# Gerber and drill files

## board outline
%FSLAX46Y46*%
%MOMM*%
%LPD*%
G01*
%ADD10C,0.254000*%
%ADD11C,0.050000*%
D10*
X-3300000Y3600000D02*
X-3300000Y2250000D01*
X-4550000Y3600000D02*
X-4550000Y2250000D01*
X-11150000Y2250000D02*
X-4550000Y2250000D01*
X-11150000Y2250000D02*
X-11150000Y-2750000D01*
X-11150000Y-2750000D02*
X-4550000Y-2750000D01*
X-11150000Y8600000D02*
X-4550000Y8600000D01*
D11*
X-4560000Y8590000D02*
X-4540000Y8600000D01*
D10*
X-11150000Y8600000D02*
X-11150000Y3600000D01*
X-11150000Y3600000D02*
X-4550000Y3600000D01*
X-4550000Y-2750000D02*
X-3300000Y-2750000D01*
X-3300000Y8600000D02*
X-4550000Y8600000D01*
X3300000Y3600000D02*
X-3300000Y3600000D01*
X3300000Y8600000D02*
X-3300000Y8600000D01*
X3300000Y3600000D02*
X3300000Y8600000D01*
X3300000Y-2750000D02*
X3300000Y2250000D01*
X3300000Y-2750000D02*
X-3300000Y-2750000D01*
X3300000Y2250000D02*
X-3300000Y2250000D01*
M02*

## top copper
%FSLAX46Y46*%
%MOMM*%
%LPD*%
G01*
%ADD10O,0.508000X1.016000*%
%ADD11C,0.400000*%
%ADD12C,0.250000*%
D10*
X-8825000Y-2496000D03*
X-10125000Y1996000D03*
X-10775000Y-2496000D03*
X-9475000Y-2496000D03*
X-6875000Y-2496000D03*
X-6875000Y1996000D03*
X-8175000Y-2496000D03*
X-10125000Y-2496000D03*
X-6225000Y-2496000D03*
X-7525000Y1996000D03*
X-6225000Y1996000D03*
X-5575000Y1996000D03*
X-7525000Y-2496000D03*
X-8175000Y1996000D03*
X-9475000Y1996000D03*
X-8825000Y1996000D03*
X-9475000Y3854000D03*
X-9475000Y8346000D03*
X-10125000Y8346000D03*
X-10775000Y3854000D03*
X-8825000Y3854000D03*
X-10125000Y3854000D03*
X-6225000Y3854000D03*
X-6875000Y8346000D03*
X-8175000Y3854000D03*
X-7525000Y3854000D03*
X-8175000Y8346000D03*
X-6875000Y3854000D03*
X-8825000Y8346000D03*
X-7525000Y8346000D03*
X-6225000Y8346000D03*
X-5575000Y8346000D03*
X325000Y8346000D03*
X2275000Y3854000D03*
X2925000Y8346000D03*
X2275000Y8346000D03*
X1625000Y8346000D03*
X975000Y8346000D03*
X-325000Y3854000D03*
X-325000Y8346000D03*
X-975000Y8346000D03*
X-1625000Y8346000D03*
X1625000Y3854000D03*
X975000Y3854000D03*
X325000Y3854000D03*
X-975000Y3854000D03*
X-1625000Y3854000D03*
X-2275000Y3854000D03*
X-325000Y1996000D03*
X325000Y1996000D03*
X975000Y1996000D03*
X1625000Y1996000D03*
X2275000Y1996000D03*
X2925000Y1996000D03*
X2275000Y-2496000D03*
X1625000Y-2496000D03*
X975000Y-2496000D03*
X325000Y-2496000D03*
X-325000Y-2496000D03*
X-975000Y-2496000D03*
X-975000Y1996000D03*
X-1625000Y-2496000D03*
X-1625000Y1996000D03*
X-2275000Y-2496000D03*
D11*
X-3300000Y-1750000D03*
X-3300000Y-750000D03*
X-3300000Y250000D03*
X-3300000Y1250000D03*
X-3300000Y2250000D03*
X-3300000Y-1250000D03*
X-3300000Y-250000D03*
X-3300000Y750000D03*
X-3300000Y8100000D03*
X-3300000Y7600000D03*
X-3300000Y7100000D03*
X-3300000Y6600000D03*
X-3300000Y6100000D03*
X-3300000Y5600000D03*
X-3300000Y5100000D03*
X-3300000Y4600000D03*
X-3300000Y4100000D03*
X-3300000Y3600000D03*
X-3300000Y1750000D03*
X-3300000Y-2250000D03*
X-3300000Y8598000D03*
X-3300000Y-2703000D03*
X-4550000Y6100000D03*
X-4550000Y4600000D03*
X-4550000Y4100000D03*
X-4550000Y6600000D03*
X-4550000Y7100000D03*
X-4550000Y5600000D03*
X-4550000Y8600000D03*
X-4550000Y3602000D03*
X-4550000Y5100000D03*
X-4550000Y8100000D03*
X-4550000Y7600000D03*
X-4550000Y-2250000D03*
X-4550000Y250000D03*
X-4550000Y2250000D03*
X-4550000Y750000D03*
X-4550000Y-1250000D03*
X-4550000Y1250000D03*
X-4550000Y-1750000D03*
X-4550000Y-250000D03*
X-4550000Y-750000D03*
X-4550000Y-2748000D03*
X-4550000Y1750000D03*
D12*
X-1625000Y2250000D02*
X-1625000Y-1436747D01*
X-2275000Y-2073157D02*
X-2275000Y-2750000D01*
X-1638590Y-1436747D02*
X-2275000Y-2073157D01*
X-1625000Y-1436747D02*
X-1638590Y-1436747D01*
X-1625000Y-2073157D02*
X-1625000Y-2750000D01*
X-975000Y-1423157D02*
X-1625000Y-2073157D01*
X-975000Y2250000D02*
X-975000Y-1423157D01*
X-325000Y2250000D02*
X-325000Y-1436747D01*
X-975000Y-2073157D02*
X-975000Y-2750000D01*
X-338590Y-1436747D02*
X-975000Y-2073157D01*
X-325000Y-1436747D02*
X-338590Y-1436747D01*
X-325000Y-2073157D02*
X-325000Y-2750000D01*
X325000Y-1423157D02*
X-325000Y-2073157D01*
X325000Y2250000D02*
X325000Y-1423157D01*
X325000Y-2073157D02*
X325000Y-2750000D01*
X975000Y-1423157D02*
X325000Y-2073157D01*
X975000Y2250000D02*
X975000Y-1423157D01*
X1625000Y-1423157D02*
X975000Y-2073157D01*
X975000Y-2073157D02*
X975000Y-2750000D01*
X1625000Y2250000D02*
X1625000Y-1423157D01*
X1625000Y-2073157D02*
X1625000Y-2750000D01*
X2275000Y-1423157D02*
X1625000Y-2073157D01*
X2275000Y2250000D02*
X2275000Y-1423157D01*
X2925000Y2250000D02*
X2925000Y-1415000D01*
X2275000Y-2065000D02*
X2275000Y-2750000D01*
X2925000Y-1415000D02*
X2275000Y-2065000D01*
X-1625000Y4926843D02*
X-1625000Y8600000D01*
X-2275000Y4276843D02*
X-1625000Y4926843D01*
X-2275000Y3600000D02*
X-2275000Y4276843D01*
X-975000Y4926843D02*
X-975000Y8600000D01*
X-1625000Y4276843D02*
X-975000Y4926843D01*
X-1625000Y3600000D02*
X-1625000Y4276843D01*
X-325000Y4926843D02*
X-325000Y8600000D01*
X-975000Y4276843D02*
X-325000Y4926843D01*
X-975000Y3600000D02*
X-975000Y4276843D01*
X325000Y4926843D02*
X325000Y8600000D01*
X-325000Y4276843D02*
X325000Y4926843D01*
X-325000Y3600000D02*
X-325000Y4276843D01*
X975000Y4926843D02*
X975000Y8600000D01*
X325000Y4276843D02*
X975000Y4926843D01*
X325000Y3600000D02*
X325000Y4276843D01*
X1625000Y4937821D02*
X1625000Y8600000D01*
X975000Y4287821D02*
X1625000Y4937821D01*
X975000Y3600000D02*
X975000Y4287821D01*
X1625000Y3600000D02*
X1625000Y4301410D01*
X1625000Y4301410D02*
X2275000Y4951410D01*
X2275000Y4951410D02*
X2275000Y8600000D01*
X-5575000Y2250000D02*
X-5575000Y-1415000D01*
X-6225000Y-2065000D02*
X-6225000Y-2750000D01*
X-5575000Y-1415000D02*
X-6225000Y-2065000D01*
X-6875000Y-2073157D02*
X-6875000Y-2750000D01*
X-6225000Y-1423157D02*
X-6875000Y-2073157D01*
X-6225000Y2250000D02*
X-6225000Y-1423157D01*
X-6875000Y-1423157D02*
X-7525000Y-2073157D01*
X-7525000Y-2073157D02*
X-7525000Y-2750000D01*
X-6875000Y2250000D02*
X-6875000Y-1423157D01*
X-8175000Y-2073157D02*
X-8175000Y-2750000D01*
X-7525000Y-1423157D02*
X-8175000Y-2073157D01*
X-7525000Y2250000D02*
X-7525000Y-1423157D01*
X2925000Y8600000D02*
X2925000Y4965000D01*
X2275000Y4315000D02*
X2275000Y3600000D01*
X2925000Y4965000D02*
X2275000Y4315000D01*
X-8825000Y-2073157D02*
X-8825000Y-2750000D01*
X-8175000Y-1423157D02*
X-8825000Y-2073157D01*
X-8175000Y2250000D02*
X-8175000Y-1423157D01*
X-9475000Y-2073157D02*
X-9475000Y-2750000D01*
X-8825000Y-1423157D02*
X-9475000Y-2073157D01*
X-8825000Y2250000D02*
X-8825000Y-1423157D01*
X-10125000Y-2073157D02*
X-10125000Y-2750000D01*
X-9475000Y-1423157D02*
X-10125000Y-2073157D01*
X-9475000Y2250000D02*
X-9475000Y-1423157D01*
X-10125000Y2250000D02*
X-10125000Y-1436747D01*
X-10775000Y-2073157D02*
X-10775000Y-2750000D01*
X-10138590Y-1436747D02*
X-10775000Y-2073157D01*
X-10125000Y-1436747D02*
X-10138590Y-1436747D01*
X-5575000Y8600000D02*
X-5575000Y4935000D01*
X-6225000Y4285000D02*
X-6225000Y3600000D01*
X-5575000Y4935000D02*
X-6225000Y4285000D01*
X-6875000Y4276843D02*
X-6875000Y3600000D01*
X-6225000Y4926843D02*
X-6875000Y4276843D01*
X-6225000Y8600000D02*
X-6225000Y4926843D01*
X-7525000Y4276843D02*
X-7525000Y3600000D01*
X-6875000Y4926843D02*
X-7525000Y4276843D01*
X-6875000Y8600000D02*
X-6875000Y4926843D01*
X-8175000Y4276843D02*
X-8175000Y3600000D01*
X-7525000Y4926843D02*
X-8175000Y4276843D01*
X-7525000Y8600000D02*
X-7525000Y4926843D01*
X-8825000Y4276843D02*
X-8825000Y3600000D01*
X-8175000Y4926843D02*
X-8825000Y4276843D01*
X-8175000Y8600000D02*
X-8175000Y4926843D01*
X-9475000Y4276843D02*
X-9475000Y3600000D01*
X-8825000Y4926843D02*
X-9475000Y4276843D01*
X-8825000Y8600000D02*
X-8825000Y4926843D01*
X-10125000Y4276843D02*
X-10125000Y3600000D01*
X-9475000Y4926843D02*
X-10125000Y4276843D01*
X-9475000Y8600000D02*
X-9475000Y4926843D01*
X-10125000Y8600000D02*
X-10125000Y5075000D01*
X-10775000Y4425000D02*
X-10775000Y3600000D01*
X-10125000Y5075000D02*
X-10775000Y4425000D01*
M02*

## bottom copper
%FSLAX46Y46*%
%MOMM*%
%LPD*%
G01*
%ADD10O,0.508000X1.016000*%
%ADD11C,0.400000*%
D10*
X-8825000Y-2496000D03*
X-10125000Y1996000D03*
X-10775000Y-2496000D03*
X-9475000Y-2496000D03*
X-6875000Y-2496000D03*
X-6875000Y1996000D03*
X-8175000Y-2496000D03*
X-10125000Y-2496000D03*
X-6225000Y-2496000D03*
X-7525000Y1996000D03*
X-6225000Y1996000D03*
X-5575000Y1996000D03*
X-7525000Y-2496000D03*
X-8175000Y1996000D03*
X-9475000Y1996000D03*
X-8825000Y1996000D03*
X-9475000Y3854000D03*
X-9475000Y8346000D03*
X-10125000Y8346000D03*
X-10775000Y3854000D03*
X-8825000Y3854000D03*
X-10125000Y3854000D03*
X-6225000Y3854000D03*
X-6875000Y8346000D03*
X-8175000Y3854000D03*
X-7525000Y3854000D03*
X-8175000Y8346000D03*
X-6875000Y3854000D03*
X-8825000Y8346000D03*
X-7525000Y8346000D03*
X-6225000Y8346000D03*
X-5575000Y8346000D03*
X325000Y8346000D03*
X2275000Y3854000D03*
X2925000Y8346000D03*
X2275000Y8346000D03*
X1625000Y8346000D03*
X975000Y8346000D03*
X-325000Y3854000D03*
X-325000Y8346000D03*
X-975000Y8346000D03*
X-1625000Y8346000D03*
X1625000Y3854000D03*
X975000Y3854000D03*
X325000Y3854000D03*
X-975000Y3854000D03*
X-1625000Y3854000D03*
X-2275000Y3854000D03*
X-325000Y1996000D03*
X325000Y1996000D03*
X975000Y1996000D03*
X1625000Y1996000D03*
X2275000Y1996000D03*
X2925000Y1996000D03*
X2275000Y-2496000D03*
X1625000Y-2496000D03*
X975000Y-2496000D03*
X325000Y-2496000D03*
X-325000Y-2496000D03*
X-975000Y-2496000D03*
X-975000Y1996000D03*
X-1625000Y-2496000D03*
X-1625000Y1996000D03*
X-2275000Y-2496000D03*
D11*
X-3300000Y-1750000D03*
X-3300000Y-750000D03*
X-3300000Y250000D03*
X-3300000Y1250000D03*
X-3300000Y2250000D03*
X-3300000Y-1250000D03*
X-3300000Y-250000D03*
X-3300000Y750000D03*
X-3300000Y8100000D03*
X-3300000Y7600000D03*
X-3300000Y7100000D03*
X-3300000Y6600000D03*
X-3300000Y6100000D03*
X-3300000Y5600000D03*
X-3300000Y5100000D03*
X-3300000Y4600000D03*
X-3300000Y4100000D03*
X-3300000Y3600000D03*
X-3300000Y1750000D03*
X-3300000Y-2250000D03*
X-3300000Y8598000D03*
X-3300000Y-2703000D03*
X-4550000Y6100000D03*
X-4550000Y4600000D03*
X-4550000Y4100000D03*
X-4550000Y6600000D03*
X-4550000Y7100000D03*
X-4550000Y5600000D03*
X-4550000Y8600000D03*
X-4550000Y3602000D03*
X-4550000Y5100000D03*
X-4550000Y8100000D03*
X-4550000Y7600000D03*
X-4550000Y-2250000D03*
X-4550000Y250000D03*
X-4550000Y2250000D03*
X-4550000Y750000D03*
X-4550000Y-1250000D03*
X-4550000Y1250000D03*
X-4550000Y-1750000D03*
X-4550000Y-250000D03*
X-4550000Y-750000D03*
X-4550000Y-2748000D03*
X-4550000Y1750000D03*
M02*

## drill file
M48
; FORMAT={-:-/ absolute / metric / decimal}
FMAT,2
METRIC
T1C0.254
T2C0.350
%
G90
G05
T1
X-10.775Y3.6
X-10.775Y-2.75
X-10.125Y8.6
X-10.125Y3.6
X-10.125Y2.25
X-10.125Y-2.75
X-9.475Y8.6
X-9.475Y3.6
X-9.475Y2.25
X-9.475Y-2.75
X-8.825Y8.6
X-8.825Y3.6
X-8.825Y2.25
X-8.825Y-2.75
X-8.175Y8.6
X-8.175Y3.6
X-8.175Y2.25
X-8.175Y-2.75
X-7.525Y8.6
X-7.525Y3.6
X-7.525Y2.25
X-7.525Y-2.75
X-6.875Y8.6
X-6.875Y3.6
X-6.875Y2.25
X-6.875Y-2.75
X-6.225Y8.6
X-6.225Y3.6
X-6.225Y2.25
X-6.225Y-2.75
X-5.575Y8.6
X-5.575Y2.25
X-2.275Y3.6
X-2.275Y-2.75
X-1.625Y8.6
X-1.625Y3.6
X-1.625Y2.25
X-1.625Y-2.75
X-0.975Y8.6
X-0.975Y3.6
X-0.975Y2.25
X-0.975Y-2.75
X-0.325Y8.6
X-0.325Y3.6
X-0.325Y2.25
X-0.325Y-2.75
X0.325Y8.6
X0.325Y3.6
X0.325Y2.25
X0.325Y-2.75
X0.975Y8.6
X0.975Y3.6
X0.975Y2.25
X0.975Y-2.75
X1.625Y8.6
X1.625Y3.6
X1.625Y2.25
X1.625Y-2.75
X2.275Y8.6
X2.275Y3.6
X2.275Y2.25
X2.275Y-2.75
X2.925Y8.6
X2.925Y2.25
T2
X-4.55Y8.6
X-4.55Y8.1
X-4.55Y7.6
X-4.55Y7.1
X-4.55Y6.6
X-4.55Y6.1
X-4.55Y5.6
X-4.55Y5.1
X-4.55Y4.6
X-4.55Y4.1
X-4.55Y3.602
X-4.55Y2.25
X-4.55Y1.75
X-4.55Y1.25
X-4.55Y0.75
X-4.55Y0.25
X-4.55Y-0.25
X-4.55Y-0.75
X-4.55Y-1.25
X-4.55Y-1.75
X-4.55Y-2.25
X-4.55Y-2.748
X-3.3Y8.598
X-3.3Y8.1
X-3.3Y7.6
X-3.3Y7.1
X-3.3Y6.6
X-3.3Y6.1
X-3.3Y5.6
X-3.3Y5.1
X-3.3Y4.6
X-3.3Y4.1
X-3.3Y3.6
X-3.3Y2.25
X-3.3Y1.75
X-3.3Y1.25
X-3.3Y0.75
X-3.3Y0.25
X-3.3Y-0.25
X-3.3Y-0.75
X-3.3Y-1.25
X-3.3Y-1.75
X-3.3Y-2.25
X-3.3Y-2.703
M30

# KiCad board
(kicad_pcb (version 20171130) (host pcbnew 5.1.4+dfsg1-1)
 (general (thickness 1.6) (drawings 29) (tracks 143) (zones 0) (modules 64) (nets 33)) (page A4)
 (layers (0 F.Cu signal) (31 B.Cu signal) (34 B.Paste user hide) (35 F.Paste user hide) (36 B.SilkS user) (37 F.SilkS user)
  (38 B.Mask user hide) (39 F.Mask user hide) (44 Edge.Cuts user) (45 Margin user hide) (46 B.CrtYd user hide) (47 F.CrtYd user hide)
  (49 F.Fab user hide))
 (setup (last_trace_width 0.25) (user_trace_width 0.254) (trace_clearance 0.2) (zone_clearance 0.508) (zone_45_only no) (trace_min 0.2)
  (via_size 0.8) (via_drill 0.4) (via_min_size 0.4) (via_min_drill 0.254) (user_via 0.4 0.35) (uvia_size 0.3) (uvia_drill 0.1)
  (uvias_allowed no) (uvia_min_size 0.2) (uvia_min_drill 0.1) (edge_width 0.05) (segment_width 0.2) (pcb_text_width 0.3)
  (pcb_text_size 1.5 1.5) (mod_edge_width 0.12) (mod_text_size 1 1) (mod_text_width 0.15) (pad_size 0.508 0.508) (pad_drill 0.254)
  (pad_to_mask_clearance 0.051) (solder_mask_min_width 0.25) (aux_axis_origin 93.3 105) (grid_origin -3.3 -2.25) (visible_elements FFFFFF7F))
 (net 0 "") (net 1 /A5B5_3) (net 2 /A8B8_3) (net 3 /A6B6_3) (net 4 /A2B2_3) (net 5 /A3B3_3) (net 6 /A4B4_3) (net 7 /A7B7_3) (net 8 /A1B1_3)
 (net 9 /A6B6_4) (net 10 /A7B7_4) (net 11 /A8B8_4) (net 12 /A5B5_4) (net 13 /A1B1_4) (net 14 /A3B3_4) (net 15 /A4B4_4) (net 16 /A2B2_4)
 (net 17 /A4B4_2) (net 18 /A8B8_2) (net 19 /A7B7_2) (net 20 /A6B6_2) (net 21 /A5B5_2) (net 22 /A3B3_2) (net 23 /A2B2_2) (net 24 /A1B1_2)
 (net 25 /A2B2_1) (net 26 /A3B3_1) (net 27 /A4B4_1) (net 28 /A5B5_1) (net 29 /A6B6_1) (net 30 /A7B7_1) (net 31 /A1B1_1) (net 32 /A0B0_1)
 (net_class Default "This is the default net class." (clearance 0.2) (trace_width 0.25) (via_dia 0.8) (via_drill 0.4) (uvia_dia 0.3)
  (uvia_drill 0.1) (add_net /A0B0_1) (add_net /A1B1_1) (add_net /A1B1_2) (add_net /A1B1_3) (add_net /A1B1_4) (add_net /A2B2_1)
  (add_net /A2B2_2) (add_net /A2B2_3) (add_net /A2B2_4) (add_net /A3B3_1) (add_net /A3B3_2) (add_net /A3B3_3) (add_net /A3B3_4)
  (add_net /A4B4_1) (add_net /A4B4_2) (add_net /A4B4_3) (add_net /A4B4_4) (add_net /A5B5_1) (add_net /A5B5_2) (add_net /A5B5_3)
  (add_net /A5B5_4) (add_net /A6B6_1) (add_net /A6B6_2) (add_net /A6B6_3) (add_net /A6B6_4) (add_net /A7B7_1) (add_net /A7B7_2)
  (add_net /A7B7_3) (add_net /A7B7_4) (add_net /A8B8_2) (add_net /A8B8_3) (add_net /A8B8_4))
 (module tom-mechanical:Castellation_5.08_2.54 (layer F.Cu) (at -8.825 2.75 180)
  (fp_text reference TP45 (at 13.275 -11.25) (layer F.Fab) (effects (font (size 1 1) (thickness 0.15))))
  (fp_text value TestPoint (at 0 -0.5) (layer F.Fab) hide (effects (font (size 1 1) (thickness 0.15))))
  (pad 1 thru_hole oval (at 0 0 180) (size 0.508 1.016) (drill 0.254 (offset 0 0.254)) (layers *.Cu *.Mask) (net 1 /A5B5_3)))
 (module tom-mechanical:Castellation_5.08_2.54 (layer F.Cu) (at -10.125 -2.25)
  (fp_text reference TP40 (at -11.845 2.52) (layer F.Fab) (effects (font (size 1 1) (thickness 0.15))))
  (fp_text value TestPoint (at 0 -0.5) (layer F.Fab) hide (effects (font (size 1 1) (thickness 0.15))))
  (pad 1 thru_hole oval (at 0 0) (size 0.508 1.016) (drill 0.254 (offset 0 0.254)) (layers *.Cu *.Mask) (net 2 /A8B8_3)))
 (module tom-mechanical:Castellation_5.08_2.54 (layer F.Cu) (at -10.775 2.75 180)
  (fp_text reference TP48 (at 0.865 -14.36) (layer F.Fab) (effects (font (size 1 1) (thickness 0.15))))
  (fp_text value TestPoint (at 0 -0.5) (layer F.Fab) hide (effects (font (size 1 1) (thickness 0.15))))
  (pad 1 thru_hole oval (at 0 0 180) (size 0.508 1.016) (drill 0.254 (offset 0 0.254)) (layers *.Cu *.Mask) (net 2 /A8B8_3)))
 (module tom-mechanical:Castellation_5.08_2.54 (layer F.Cu) (at -9.475 2.75 180)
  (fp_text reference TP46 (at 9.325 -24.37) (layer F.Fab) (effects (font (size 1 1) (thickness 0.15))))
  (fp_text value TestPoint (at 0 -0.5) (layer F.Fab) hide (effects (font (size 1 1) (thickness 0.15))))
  (pad 1 thru_hole oval (at 0 0 180) (size 0.508 1.016) (drill 0.254 (offset 0 0.254)) (layers *.Cu *.Mask) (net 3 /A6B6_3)))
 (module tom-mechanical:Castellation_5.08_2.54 (layer F.Cu) (at -6.875 2.75 180)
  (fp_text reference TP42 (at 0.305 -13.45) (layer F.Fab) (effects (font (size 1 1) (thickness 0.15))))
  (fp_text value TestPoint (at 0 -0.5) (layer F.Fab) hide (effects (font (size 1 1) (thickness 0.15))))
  (pad 1 thru_hole oval (at 0 0 180) (size 0.508 1.016) (drill 0.254 (offset 0 0.254)) (layers *.Cu *.Mask) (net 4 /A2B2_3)))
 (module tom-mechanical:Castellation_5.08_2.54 (layer F.Cu) (at -6.875 -2.25)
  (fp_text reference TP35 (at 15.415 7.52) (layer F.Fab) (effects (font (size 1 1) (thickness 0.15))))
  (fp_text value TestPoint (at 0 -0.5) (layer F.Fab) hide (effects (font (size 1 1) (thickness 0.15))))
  (pad 1 thru_hole oval (at 0 0) (size 0.508 1.016) (drill 0.254 (offset 0 0.254)) (layers *.Cu *.Mask) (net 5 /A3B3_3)))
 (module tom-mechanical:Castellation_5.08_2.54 (layer F.Cu) (at -8.175 2.75 180)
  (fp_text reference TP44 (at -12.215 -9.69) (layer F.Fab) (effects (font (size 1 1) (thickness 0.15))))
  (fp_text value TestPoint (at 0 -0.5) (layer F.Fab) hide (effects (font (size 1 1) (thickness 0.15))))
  (pad 1 thru_hole oval (at 0 0 180) (size 0.508 1.016) (drill 0.254 (offset 0 0.254)) (layers *.Cu *.Mask) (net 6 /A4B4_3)))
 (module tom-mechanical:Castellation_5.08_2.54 (layer F.Cu) (at -10.125 2.75 180)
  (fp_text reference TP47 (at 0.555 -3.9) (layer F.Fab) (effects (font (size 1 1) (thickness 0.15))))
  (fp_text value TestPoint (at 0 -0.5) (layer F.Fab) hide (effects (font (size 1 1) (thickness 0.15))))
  (pad 1 thru_hole oval (at 0 0 180) (size 0.508 1.016) (drill 0.254 (offset 0 0.254)) (layers *.Cu *.Mask) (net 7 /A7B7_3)))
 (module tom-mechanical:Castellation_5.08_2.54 (layer F.Cu) (at -6.225 2.75 180)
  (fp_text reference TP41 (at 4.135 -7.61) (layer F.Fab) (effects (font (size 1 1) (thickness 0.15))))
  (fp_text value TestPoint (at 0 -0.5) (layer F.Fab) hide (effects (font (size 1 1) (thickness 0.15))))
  (pad 1 thru_hole oval (at 0 0 180) (size 0.508 1.016) (drill 0.254 (offset 0 0.254)) (layers *.Cu *.Mask) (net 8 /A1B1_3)))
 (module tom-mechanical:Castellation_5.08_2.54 (layer F.Cu) (at -7.525 -2.25)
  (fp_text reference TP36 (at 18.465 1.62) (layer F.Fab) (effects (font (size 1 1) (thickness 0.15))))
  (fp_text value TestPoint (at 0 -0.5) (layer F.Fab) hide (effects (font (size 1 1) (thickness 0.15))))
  (pad 1 thru_hole oval (at 0 0) (size 0.508 1.016) (drill 0.254 (offset 0 0.254)) (layers *.Cu *.Mask) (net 6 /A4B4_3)))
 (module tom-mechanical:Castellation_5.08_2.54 (layer F.Cu) (at -6.225 -2.25)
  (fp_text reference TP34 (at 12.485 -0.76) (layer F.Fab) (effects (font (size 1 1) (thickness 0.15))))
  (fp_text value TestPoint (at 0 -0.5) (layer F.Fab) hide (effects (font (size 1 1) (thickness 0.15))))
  (pad 1 thru_hole oval (at 0 0) (size 0.508 1.016) (drill 0.254 (offset 0 0.254)) (layers *.Cu *.Mask) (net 4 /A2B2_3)))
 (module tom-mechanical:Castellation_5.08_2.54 (layer F.Cu) (at -5.575 -2.25)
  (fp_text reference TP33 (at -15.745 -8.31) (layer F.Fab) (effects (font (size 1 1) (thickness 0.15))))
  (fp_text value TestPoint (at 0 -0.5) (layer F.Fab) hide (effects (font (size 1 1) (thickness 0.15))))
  (pad 1 thru_hole oval (at 0 0) (size 0.508 1.016) (drill 0.254 (offset 0 0.254)) (layers *.Cu *.Mask) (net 8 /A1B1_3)))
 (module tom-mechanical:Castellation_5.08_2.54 (layer F.Cu) (at -7.525 2.75 180)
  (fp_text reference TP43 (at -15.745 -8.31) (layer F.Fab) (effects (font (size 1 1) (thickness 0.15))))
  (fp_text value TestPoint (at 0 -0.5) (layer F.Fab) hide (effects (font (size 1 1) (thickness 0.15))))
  (pad 1 thru_hole oval (at 0 0 180) (size 0.508 1.016) (drill 0.254 (offset 0 0.254)) (layers *.Cu *.Mask) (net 5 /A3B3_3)))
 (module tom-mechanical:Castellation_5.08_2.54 (layer F.Cu) (at -8.175 -2.25)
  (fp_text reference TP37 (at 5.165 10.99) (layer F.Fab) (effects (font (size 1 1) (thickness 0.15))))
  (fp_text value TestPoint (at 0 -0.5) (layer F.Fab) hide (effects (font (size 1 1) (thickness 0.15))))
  (pad 1 thru_hole oval (at 0 0) (size 0.508 1.016) (drill 0.254 (offset 0 0.254)) (layers *.Cu *.Mask) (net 1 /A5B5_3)))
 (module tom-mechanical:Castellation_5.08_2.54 (layer F.Cu) (at -9.475 -2.25)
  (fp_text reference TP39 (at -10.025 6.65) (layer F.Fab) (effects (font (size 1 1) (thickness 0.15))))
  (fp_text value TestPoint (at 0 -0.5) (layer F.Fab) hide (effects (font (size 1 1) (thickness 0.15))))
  (pad 1 thru_hole oval (at 0 0) (size 0.508 1.016) (drill 0.254 (offset 0 0.254)) (layers *.Cu *.Mask) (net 7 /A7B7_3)))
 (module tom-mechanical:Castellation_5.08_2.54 (layer F.Cu) (at -8.825 -2.25)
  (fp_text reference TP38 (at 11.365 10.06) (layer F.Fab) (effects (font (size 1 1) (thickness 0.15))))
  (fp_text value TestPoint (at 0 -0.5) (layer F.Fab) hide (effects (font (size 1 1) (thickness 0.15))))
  (pad 1 thru_hole oval (at 0 0) (size 0.508 1.016) (drill 0.254 (offset 0 0.254)) (layers *.Cu *.Mask) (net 3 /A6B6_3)))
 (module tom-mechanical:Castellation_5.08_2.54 (layer F.Cu) (at -9.475 -3.6 180)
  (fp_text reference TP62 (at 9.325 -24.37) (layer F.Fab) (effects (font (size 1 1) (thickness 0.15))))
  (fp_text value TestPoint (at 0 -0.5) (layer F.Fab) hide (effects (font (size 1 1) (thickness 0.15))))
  (pad 1 thru_hole oval (at 0 0 180) (size 0.508 1.016) (drill 0.254 (offset 0 0.254)) (layers *.Cu *.Mask) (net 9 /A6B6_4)))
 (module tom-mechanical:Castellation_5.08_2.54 (layer F.Cu) (at -9.475 -8.6)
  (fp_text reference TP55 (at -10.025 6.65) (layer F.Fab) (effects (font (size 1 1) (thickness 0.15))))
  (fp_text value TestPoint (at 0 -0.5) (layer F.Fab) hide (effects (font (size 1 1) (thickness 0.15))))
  (pad 1 thru_hole oval (at 0 0) (size 0.508 1.016) (drill 0.254 (offset 0 0.254)) (layers *.Cu *.Mask) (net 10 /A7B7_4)))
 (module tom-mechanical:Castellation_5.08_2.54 (layer F.Cu) (at -10.125 -8.6)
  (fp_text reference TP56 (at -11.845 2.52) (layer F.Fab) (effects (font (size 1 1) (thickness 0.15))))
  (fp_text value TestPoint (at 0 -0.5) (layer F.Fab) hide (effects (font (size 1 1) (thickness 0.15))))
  (pad 1 thru_hole oval (at 0 0) (size 0.508 1.016) (drill 0.254 (offset 0 0.254)) (layers *.Cu *.Mask) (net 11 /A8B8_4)))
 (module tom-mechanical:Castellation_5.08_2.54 (layer F.Cu) (at -10.775 -3.6 180)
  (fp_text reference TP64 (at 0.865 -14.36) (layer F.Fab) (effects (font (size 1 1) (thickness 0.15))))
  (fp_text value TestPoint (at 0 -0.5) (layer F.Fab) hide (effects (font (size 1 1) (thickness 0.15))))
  (pad 1 thru_hole oval (at 0 0 180) (size 0.508 1.016) (drill 0.254 (offset 0 0.254)) (layers *.Cu *.Mask) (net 11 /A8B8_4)))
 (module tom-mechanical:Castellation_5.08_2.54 (layer F.Cu) (at -8.825 -3.6 180)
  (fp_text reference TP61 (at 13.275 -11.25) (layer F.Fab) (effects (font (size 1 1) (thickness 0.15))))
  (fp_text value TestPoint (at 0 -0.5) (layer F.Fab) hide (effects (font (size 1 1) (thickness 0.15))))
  (pad 1 thru_hole oval (at 0 0 180) (size 0.508 1.016) (drill 0.254 (offset 0 0.254)) (layers *.Cu *.Mask) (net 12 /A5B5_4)))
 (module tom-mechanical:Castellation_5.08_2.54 (layer F.Cu) (at -10.125 -3.6 180)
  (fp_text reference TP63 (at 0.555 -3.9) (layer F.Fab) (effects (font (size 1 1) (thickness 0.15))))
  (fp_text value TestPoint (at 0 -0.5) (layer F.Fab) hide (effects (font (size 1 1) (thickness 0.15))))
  (pad 1 thru_hole oval (at 0 0 180) (size 0.508 1.016) (drill 0.254 (offset 0 0.254)) (layers *.Cu *.Mask) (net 10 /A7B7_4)))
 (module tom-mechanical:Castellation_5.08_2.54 (layer F.Cu) (at -6.225 -3.6 180)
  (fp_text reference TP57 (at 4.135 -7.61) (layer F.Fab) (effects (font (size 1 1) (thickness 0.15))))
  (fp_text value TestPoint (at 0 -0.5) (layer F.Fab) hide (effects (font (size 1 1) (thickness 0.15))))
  (pad 1 thru_hole oval (at 0 0 180) (size 0.508 1.016) (drill 0.254 (offset 0 0.254)) (layers *.Cu *.Mask) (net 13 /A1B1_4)))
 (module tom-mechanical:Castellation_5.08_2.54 (layer F.Cu) (at -6.875 -8.6)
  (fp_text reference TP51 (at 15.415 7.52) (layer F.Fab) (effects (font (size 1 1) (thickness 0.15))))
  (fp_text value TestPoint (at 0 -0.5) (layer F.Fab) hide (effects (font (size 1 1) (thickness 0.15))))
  (pad 1 thru_hole oval (at 0 0) (size 0.508 1.016) (drill 0.254 (offset 0 0.254)) (layers *.Cu *.Mask) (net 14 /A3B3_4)))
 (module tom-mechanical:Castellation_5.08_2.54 (layer F.Cu) (at -8.175 -3.6 180)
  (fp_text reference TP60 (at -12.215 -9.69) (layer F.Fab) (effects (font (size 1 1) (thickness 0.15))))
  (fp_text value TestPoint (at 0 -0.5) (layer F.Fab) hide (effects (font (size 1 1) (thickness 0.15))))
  (pad 1 thru_hole oval (at 0 0 180) (size 0.508 1.016) (drill 0.254 (offset 0 0.254)) (layers *.Cu *.Mask) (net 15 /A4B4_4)))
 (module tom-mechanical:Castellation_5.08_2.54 (layer F.Cu) (at -7.525 -3.6 180)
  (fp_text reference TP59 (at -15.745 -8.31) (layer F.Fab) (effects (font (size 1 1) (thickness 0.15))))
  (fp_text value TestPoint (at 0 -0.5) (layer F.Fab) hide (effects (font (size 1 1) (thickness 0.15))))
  (pad 1 thru_hole oval (at 0 0 180) (size 0.508 1.016) (drill 0.254 (offset 0 0.254)) (layers *.Cu *.Mask) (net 14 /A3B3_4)))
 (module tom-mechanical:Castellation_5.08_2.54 (layer F.Cu) (at -8.175 -8.6)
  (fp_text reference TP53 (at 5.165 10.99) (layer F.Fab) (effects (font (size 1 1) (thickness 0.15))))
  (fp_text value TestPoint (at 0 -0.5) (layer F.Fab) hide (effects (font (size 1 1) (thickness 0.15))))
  (pad 1 thru_hole oval (at 0 0) (size 0.508 1.016) (drill 0.254 (offset 0 0.254)) (layers *.Cu *.Mask) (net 12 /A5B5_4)))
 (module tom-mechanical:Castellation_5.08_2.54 (layer F.Cu) (at -6.875 -3.6 180)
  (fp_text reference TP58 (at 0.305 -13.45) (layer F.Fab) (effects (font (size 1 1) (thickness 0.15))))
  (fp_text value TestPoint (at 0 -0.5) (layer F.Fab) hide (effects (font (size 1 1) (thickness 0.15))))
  (pad 1 thru_hole oval (at 0 0 180) (size 0.508 1.016) (drill 0.254 (offset 0 0.254)) (layers *.Cu *.Mask) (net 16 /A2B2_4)))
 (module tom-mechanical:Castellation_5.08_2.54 (layer F.Cu) (at -8.825 -8.6)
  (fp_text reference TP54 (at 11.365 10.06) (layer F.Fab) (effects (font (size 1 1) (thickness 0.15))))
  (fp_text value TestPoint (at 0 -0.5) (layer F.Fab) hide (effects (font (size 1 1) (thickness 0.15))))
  (pad 1 thru_hole oval (at 0 0) (size 0.508 1.016) (drill 0.254 (offset 0 0.254)) (layers *.Cu *.Mask) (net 9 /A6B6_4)))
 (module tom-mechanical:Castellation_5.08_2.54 (layer F.Cu) (at -7.525 -8.6)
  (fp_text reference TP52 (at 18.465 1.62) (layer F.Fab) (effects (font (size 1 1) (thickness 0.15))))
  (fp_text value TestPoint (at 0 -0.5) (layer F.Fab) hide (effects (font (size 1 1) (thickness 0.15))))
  (pad 1 thru_hole oval (at 0 0) (size 0.508 1.016) (drill 0.254 (offset 0 0.254)) (layers *.Cu *.Mask) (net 15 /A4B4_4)))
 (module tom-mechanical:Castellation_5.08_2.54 (layer F.Cu) (at -6.225 -8.6)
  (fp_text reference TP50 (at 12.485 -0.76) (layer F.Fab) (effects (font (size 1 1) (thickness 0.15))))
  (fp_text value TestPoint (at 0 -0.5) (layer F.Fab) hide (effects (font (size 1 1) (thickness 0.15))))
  (pad 1 thru_hole oval (at 0 0) (size 0.508 1.016) (drill 0.254 (offset 0 0.254)) (layers *.Cu *.Mask) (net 16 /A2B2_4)))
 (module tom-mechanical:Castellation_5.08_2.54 (layer F.Cu) (at -5.575 -8.6)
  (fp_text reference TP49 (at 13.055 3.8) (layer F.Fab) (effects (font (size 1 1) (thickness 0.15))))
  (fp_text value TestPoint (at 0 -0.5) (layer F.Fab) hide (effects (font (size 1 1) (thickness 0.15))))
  (pad 1 thru_hole oval (at 0 0) (size 0.508 1.016) (drill 0.254 (offset 0 0.254)) (layers *.Cu *.Mask) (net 13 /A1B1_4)))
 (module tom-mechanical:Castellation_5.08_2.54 (layer F.Cu) (at 0.325 -8.6)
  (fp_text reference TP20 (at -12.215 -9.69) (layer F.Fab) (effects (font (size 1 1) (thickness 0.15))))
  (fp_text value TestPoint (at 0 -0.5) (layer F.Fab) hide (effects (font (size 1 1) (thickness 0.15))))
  (pad 1 thru_hole oval (at 0 0) (size 0.508 1.016) (drill 0.254 (offset 0 0.254)) (layers *.Cu *.Mask) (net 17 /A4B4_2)))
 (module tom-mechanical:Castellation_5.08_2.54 (layer F.Cu) (at 2.275 -3.6 180)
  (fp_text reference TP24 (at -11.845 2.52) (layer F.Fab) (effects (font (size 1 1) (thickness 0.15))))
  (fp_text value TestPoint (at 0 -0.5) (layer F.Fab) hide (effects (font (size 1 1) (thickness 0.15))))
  (pad 1 thru_hole oval (at 0 0 180) (size 0.508 1.016) (drill 0.254 (offset 0 0.254)) (layers *.Cu *.Mask) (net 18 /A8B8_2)))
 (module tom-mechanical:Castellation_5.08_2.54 (layer F.Cu) (at 2.925 -8.6)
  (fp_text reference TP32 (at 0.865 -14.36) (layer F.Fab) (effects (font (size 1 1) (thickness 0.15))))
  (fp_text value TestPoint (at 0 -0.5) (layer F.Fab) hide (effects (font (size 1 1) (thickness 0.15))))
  (pad 1 thru_hole oval (at 0 0) (size 0.508 1.016) (drill 0.254 (offset 0 0.254)) (layers *.Cu *.Mask) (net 18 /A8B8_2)))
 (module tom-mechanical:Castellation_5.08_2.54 (layer F.Cu) (at 2.275 -8.6)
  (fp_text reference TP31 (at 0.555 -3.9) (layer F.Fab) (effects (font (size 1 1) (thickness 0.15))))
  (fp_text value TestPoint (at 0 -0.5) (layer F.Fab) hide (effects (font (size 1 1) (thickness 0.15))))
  (pad 1 thru_hole oval (at 0 0) (size 0.508 1.016) (drill 0.254 (offset 0 0.254)) (layers *.Cu *.Mask) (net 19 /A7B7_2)))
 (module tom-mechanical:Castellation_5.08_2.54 (layer F.Cu) (at 1.625 -8.6)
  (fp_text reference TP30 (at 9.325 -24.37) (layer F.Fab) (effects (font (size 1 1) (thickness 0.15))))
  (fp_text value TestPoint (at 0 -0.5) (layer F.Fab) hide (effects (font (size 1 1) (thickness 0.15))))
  (pad 1 thru_hole oval (at 0 0) (size 0.508 1.016) (drill 0.254 (offset 0 0.254)) (layers *.Cu *.Mask) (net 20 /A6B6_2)))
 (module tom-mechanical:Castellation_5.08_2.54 (layer F.Cu) (at 0.975 -8.6)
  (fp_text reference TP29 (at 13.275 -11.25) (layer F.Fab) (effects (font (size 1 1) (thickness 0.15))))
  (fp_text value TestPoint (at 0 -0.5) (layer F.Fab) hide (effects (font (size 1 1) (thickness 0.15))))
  (pad 1 thru_hole oval (at 0 0) (size 0.508 1.016) (drill 0.254 (offset 0 0.254)) (layers *.Cu *.Mask) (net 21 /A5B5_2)))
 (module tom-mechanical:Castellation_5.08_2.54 (layer F.Cu) (at -0.325 -3.6 180)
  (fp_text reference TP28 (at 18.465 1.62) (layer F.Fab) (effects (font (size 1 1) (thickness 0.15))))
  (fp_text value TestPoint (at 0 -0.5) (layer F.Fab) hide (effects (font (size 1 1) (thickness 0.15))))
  (pad 1 thru_hole oval (at 0 0 180) (size 0.508 1.016) (drill 0.254 (offset 0 0.254)) (layers *.Cu *.Mask) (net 17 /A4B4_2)))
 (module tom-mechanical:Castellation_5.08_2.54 (layer F.Cu) (at -0.325 -8.6)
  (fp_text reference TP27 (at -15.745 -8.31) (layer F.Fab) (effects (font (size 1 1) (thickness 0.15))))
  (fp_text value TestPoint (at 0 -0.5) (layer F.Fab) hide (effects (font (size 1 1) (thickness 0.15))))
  (pad 1 thru_hole oval (at 0 0) (size 0.508 1.016) (drill 0.254 (offset 0 0.254)) (layers *.Cu *.Mask) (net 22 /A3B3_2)))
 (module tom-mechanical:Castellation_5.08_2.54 (layer F.Cu) (at -0.975 -8.6)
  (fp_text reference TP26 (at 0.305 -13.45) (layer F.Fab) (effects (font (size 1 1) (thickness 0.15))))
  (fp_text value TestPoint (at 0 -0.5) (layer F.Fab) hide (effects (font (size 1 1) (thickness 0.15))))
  (pad 1 thru_hole oval (at 0 0) (size 0.508 1.016) (drill 0.254 (offset 0 0.254)) (layers *.Cu *.Mask) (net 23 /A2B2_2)))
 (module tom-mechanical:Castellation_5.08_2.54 (layer F.Cu) (at -1.625 -8.6)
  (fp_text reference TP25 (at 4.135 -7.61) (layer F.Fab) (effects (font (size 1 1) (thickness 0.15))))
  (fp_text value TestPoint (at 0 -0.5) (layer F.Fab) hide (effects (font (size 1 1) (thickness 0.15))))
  (pad 1 thru_hole oval (at 0 0) (size 0.508 1.016) (drill 0.254 (offset 0 0.254)) (layers *.Cu *.Mask) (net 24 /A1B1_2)))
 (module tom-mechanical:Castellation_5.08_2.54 (layer F.Cu) (at 1.625 -3.6 180)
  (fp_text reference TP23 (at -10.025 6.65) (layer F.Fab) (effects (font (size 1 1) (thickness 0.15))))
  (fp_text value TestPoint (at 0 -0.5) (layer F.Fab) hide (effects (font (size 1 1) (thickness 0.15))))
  (pad 1 thru_hole oval (at 0 0 180) (size 0.508 1.016) (drill 0.254 (offset 0 0.254)) (layers *.Cu *.Mask) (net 19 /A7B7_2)))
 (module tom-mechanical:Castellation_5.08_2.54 (layer F.Cu) (at 0.975 -3.6 180)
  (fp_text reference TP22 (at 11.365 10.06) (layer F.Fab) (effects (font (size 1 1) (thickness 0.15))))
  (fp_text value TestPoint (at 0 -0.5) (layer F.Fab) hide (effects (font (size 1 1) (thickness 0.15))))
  (pad 1 thru_hole oval (at 0 0 180) (size 0.508 1.016) (drill 0.254 (offset 0 0.254)) (layers *.Cu *.Mask) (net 20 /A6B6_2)))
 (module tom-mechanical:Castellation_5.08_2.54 (layer F.Cu) (at 0.325 -3.6 180)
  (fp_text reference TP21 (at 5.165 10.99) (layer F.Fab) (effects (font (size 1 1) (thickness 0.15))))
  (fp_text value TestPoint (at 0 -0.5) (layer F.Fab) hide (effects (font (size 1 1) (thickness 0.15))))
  (pad 1 thru_hole oval (at 0 0 180) (size 0.508 1.016) (drill 0.254 (offset 0 0.254)) (layers *.Cu *.Mask) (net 21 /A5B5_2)))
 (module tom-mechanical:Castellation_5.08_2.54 (layer F.Cu) (at -0.975 -3.6 180)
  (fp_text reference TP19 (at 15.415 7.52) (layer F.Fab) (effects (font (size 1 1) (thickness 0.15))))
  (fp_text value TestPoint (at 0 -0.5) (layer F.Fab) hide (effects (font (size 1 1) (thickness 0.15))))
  (pad 1 thru_hole oval (at 0 0 180) (size 0.508 1.016) (drill 0.254 (offset 0 0.254)) (layers *.Cu *.Mask) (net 22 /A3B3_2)))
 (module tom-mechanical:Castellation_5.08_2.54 (layer F.Cu) (at -1.625 -3.6 180)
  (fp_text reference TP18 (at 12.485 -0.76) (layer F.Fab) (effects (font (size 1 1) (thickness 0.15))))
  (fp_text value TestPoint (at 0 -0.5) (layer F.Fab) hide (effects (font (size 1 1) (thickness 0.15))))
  (pad 1 thru_hole oval (at 0 0 180) (size 0.508 1.016) (drill 0.254 (offset 0 0.254)) (layers *.Cu *.Mask) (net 23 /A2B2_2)))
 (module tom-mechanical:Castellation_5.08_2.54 (layer F.Cu) (at -2.275 -3.6 180)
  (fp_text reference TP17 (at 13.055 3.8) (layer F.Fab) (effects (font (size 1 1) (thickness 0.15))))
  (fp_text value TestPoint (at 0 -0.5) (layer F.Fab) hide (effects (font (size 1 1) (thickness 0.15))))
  (pad 1 thru_hole oval (at 0 0 180) (size 0.508 1.016) (drill 0.254 (offset 0 0.254)) (layers *.Cu *.Mask) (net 24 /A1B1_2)))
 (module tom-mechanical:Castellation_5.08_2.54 (layer F.Cu) (at -0.325 -2.25)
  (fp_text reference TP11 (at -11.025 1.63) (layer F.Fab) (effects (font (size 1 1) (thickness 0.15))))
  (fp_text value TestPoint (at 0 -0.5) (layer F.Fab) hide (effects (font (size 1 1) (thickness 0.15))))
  (pad 1 thru_hole oval (at 0 0) (size 0.508 1.016) (drill 0.254 (offset 0 0.254)) (layers *.Cu *.Mask) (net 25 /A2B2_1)))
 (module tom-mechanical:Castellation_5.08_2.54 (layer F.Cu) (at 0.325 -2.25)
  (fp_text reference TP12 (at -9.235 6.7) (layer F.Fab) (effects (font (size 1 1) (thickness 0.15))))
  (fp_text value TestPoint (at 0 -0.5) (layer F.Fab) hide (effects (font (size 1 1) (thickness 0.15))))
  (pad 1 thru_hole oval (at 0 0) (size 0.508 1.016) (drill 0.254 (offset 0 0.254)) (layers *.Cu *.Mask) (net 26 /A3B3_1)))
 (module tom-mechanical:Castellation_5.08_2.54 (layer F.Cu) (at 0.975 -2.25)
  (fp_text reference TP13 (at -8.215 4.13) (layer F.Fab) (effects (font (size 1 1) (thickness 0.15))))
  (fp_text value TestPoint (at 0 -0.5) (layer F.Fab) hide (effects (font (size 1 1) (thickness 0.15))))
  (pad 1 thru_hole oval (at 0 0) (size 0.508 1.016) (drill 0.254 (offset 0 0.254)) (layers *.Cu *.Mask) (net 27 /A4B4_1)))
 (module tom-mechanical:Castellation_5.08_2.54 (layer F.Cu) (at 1.625 -2.25)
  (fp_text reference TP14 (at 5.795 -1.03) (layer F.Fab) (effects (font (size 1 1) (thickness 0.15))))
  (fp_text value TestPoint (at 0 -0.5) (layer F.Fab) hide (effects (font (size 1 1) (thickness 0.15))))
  (pad 1 thru_hole oval (at 0 0) (size 0.508 1.016) (drill 0.254 (offset 0 0.254)) (layers *.Cu *.Mask) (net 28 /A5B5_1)))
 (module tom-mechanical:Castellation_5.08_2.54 (layer F.Cu) (at 2.275 -2.25)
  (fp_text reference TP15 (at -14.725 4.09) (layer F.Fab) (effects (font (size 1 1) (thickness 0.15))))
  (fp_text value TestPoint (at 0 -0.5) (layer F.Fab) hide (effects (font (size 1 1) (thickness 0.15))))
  (pad 1 thru_hole oval (at 0 0) (size 0.508 1.016) (drill 0.254 (offset 0 0.254)) (layers *.Cu *.Mask) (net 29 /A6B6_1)))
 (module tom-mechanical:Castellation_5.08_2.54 (layer F.Cu) (at 2.925 -2.25)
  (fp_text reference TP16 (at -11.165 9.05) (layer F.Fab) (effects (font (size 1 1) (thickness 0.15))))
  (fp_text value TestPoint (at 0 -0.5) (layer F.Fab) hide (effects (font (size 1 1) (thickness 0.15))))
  (pad 1 thru_hole oval (at 0 0) (size 0.508 1.016) (drill 0.254 (offset 0 0.254)) (layers *.Cu *.Mask) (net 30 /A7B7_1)))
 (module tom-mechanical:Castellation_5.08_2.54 (layer F.Cu) (at 2.275 2.75 180)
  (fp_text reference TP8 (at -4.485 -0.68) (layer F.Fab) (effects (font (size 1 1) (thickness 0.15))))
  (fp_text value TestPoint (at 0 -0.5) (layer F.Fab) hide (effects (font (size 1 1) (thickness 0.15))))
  (pad 1 thru_hole oval (at 0 0 180) (size 0.508 1.016) (drill 0.254 (offset 0 0.254)) (layers *.Cu *.Mask) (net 30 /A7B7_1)))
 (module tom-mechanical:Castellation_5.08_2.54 (layer F.Cu) (at 1.625 2.75 180)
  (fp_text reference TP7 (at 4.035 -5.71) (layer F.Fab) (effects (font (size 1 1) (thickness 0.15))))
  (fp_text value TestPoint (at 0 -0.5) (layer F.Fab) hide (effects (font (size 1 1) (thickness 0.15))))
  (pad 1 thru_hole oval (at 0 0 180) (size 0.508 1.016) (drill 0.254 (offset 0 0.254)) (layers *.Cu *.Mask) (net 29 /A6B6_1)))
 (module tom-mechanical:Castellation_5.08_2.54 (layer F.Cu) (at 0.975 2.75 180)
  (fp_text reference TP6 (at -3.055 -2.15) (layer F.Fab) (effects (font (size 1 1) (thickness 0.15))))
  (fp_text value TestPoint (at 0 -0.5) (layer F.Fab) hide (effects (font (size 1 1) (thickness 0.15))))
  (pad 1 thru_hole oval (at 0 0 180) (size 0.508 1.016) (drill 0.254 (offset 0 0.254)) (layers *.Cu *.Mask) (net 28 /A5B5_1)))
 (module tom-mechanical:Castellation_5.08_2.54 (layer F.Cu) (at 0.325 2.75 180)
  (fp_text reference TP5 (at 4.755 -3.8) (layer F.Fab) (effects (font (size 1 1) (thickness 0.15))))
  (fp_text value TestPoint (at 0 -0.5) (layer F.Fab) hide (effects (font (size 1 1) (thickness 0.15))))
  (pad 1 thru_hole oval (at 0 0 180) (size 0.508 1.016) (drill 0.254 (offset 0 0.254)) (layers *.Cu *.Mask) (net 27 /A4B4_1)))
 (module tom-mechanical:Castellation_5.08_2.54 (layer F.Cu) (at -0.325 2.75 180)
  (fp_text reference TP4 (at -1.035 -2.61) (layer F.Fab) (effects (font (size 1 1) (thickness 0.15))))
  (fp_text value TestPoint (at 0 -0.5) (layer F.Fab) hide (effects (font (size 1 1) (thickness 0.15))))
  (pad 1 thru_hole oval (at 0 0 180) (size 0.508 1.016) (drill 0.254 (offset 0 0.254)) (layers *.Cu *.Mask) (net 26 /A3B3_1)))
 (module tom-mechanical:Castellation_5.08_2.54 (layer F.Cu) (at -0.975 2.75 180)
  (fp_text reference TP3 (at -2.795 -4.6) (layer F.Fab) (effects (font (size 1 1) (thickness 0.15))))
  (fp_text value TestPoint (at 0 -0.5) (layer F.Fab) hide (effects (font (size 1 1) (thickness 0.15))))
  (pad 1 thru_hole oval (at 0 0 180) (size 0.508 1.016) (drill 0.254 (offset 0 0.254)) (layers *.Cu *.Mask) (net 25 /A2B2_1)))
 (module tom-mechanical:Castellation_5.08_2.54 (layer F.Cu) (at -0.975 -2.25)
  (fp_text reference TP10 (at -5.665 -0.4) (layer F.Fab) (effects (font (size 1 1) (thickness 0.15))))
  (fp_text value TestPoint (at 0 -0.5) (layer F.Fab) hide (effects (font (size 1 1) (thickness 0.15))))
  (pad 1 thru_hole oval (at 0 0) (size 0.508 1.016) (drill 0.254 (offset 0 0.254)) (layers *.Cu *.Mask) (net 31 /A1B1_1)))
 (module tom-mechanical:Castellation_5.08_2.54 (layer F.Cu) (at -1.625 2.75 180)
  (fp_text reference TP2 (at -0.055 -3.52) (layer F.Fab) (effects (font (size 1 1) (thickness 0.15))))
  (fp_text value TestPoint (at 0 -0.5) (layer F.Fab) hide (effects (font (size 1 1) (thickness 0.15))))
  (pad 1 thru_hole oval (at 0 0 180) (size 0.508 1.016) (drill 0.254 (offset 0 0.254)) (layers *.Cu *.Mask) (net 31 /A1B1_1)))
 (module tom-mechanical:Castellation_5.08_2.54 (layer F.Cu) (at -1.625 -2.25)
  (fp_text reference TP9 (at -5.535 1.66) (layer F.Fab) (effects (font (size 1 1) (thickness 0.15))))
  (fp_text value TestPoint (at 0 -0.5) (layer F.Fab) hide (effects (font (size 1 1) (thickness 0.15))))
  (pad 1 thru_hole oval (at 0 0) (size 0.508 1.016) (drill 0.254 (offset 0 0.254)) (layers *.Cu *.Mask) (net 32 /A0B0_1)))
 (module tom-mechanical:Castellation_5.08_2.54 (layer F.Cu) (at -2.275 2.75 180)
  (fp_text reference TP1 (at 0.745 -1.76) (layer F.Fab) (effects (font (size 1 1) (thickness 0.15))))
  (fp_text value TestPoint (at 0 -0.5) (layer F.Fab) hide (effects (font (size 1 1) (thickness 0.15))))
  (pad 1 thru_hole oval (at 0 0 180) (size 0.508 1.016) (drill 0.254 (offset 0 0.254)) (layers *.Cu *.Mask) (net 32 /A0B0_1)))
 (gr_line (start -3.3 -3.6) (end -3.3 -2.25) (layer Edge.Cuts) (width 0.254))
 (gr_line (start -4.55 -3.6) (end -4.55 -2.25) (layer Edge.Cuts) (width 0.254))
 (gr_line (start -11.15 -2.25) (end -4.55 -2.25) (layer Edge.Cuts) (width 0.254))
 (gr_line (start -11.15 -2.25) (end -11.15 2.75) (layer Edge.Cuts) (width 0.254))
 (gr_line (start -11.15 2.75) (end -4.55 2.75) (layer Edge.Cuts) (width 0.254))
 (gr_line (start -11.15 -8.6) (end -4.55 -8.6) (layer Edge.Cuts) (width 0.254))
 (gr_line (start -4.56 -8.59) (end -4.54 -8.6) (layer Edge.Cuts) (width 0.05))
 (gr_line (start -11.15 -8.6) (end -11.15 -3.6) (layer Edge.Cuts) (width 0.254))
 (gr_line (start -11.15 -3.6) (end -4.55 -3.6) (layer Edge.Cuts) (width 0.254))
 (gr_line (start -4.55 2.75) (end -3.3 2.75) (layer Edge.Cuts) (width 0.254))
 (gr_line (start -3.3 -8.6) (end -4.55 -8.6) (layer Edge.Cuts) (width 0.254))
 (gr_line (start 3.3 -3.6) (end -3.3 -3.6) (layer Edge.Cuts) (width 0.254))
 (gr_line (start 3.3 -8.6) (end -3.3 -8.6) (layer Edge.Cuts) (width 0.254))
 (gr_line (start 3.3 -3.6) (end 3.3 -8.6) (layer Edge.Cuts) (width 0.254))
 (gr_line (start 3.3 2.75) (end 3.3 -2.25) (layer Edge.Cuts) (width 0.254))
 (gr_line (start 3.3 2.75) (end -3.3 2.75) (layer Edge.Cuts) (width 0.254))
 (gr_line (start 3.3 -2.25) (end -3.3 -2.25) (layer Edge.Cuts) (width 0.254))
 (via (at -3.3 1.75) (size 0.4) (drill 0.35) (layers F.Cu B.Cu) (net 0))
 (via (at -3.3 0.75) (size 0.4) (drill 0.35) (layers F.Cu B.Cu) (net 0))
 (via (at -3.3 -0.25) (size 0.4) (drill 0.35) (layers F.Cu B.Cu) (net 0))
 (via (at -3.3 -1.25) (size 0.4) (drill 0.35) (layers F.Cu B.Cu) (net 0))
 (via (at -3.3 -2.25) (size 0.4) (drill 0.35) (layers F.Cu B.Cu) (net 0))
 (via (at -3.3 1.25) (size 0.4) (drill 0.35) (layers F.Cu B.Cu) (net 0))
 (via (at -3.3 0.25) (size 0.4) (drill 0.35) (layers F.Cu B.Cu) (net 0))
 (via (at -3.3 -0.75) (size 0.4) (drill 0.35) (layers F.Cu B.Cu) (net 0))
 (via (at -3.3 -8.1) (size 0.4) (drill 0.35) (layers F.Cu B.Cu) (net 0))
 (via (at -3.3 -7.6) (size 0.4) (drill 0.35) (layers F.Cu B.Cu) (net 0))
 (via (at -3.3 -7.1) (size 0.4) (drill 0.35) (layers F.Cu B.Cu) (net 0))
 (via (at -3.3 -6.6) (size 0.4) (drill 0.35) (layers F.Cu B.Cu) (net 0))
 (via (at -3.3 -6.1) (size 0.4) (drill 0.35) (layers F.Cu B.Cu) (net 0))
 (via (at -3.3 -5.6) (size 0.4) (drill 0.35) (layers F.Cu B.Cu) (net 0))
 (via (at -3.3 -5.1) (size 0.4) (drill 0.35) (layers F.Cu B.Cu) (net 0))
 (via (at -3.3 -4.6) (size 0.4) (drill 0.35) (layers F.Cu B.Cu) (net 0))
 (via (at -3.3 -4.1) (size 0.4) (drill 0.35) (layers F.Cu B.Cu) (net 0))
 (via (at -3.3 -3.6) (size 0.4) (drill 0.35) (layers F.Cu B.Cu) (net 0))
 (via (at -3.3 -1.75) (size 0.4) (drill 0.35) (layers F.Cu B.Cu) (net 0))
 (via (at -3.3 2.25) (size 0.4) (drill 0.35) (layers F.Cu B.Cu) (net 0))
 (via (at -3.3 -8.598) (size 0.4) (drill 0.35) (layers F.Cu B.Cu) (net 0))
 (via (at -3.3 2.703) (size 0.4) (drill 0.35) (layers F.Cu B.Cu) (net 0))
 (via (at -4.55 -6.1) (size 0.4) (drill 0.35) (layers F.Cu B.Cu) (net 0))
 (via (at -4.55 -4.6) (size 0.4) (drill 0.35) (layers F.Cu B.Cu) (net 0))
 (via (at -4.55 -4.1) (size 0.4) (drill 0.35) (layers F.Cu B.Cu) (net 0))
 (via (at -4.55 -6.6) (size 0.4) (drill 0.35) (layers F.Cu B.Cu) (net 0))
 (via (at -4.55 -7.1) (size 0.4) (drill 0.35) (layers F.Cu B.Cu) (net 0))
 (via (at -4.55 -5.6) (size 0.4) (drill 0.35) (layers F.Cu B.Cu) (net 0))
 (via (at -4.55 -8.6) (size 0.4) (drill 0.35) (layers F.Cu B.Cu) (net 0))
 (via (at -4.55 -3.602) (size 0.4) (drill 0.35) (layers F.Cu B.Cu) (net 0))
 (via (at -4.55 -5.1) (size 0.4) (drill 0.35) (layers F.Cu B.Cu) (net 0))
 (via (at -4.55 -8.1) (size 0.4) (drill 0.35) (layers F.Cu B.Cu) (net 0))
 (via (at -4.55 -7.6) (size 0.4) (drill 0.35) (layers F.Cu B.Cu) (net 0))
 (via (at -4.55 2.25) (size 0.4) (drill 0.35) (layers F.Cu B.Cu) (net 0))
 (via (at -4.55 -0.25) (size 0.4) (drill 0.35) (layers F.Cu B.Cu) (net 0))
 (via (at -4.55 -2.25) (size 0.4) (drill 0.35) (layers F.Cu B.Cu) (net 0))
 (via (at -4.55 -0.75) (size 0.4) (drill 0.35) (layers F.Cu B.Cu) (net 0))
 (via (at -4.55 1.25) (size 0.4) (drill 0.35) (layers F.Cu B.Cu) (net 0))
 (via (at -4.55 -1.25) (size 0.4) (drill 0.35) (layers F.Cu B.Cu) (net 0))
 (via (at -4.55 1.75) (size 0.4) (drill 0.35) (layers F.Cu B.Cu) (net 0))
 (via (at -4.55 0.25) (size 0.4) (drill 0.35) (layers F.Cu B.Cu) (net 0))
 (via (at -4.55 0.75) (size 0.4) (drill 0.35) (layers F.Cu B.Cu) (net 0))
 (via (at -4.55 2.748) (size 0.4) (drill 0.35) (layers F.Cu B.Cu) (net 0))
 (via (at -4.55 -1.75) (size 0.4) (drill 0.35) (layers F.Cu B.Cu) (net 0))
 (segment (start -1.625 -2.25) (end -1.625 1.436747) (width 0.25) (layer F.Cu) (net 32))
 (segment (start -2.275 2.073157) (end -2.275 2.75) (width 0.25) (layer F.Cu) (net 32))
 (segment (start -1.63859 1.436747) (end -2.275 2.073157) (width 0.25) (layer F.Cu) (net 32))
 (segment (start -1.625 1.436747) (end -1.63859 1.436747) (width 0.25) (layer F.Cu) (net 32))
 (segment (start -1.625 2.073157) (end -1.625 2.75) (width 0.25) (layer F.Cu) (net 31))
 (segment (start -0.975 1.423157) (end -1.625 2.073157) (width 0.25) (layer F.Cu) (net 31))
 (segment (start -0.975 -2.25) (end -0.975 1.423157) (width 0.25) (layer F.Cu) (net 31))
 (segment (start -0.325 -2.25) (end -0.325 1.436747) (width 0.25) (layer F.Cu) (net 25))
 (segment (start -0.975 2.073157) (end -0.975 2.75) (width 0.25) (layer F.Cu) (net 25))
 (segment (start -0.33859 1.436747) (end -0.975 2.073157) (width 0.25) (layer F.Cu) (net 25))
 (segment (start -0.325 1.436747) (end -0.33859 1.436747) (width 0.25) (layer F.Cu) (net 25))
 (segment (start -0.325 2.073157) (end -0.325 2.75) (width 0.25) (layer F.Cu) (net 26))
 (segment (start 0.325 1.423157) (end -0.325 2.073157) (width 0.25) (layer F.Cu) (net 26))
 (segment (start 0.325 -2.25) (end 0.325 1.423157) (width 0.25) (layer F.Cu) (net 26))
 (segment (start 0.325 2.073157) (end 0.325 2.75) (width 0.25) (layer F.Cu) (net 27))
 (segment (start 0.975 1.423157) (end 0.325 2.073157) (width 0.25) (layer F.Cu) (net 27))
 (segment (start 0.975 -2.25) (end 0.975 1.423157) (width 0.25) (layer F.Cu) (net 27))
 (segment (start 1.625 1.423157) (end 0.975 2.073157) (width 0.25) (layer F.Cu) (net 28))
 (segment (start 0.975 2.073157) (end 0.975 2.75) (width 0.25) (layer F.Cu) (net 28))
 (segment (start 1.625 -2.25) (end 1.625 1.423157) (width 0.25) (layer F.Cu) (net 28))
 (segment (start 1.625 2.073157) (end 1.625 2.75) (width 0.25) (layer F.Cu) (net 29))
 (segment (start 2.275 1.423157) (end 1.625 2.073157) (width 0.25) (layer F.Cu) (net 29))
 (segment (start 2.275 -2.25) (end 2.275 1.423157) (width 0.25) (layer F.Cu) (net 29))
 (segment (start 2.925 -2.25) (end 2.925 1.415) (width 0.25) (layer F.Cu) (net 30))
 (segment (start 2.275 2.065) (end 2.275 2.75) (width 0.25) (layer F.Cu) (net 30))
 (segment (start 2.925 1.415) (end 2.275 2.065) (width 0.25) (layer F.Cu) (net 30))
 (segment (start -1.625 -4.926843) (end -1.625 -8.6) (width 0.25) (layer F.Cu) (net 24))
 (segment (start -2.275 -4.276843) (end -1.625 -4.926843) (width 0.25) (layer F.Cu) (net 24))
 (segment (start -2.275 -3.6) (end -2.275 -4.276843) (width 0.25) (layer F.Cu) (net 24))
 (segment (start -0.975 -4.926843) (end -0.975 -8.6) (width 0.25) (layer F.Cu) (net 23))
 (segment (start -1.625 -4.276843) (end -0.975 -4.926843) (width 0.25) (layer F.Cu) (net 23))
 (segment (start -1.625 -3.6) (end -1.625 -4.276843) (width 0.25) (layer F.Cu) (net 23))
 (segment (start -0.325 -4.926843) (end -0.325 -8.6) (width 0.25) (layer F.Cu) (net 22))
 (segment (start -0.975 -4.276843) (end -0.325 -4.926843) (width 0.25) (layer F.Cu) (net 22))
 (segment (start -0.975 -3.6) (end -0.975 -4.276843) (width 0.25) (layer F.Cu) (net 22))
 (segment (start 0.325 -4.926843) (end 0.325 -8.6) (width 0.25) (layer F.Cu) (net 17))
 (segment (start -0.325 -4.276843) (end 0.325 -4.926843) (width 0.25) (layer F.Cu) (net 17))
 (segment (start -0.325 -3.6) (end -0.325 -4.276843) (width 0.25) (layer F.Cu) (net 17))
 (segment (start 0.975 -4.926843) (end 0.975 -8.6) (width 0.25) (layer F.Cu) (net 21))
 (segment (start 0.325 -4.276843) (end 0.975 -4.926843) (width 0.25) (layer F.Cu) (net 21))
 (segment (start 0.325 -3.6) (end 0.325 -4.276843) (width 0.25) (layer F.Cu) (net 21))
 (segment (start 1.625 -4.937821) (end 1.625 -8.6) (width 0.25) (layer F.Cu) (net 20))
 (segment (start 0.975 -4.287821) (end 1.625 -4.937821) (width 0.25) (layer F.Cu) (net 20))
 (segment (start 0.975 -3.6) (end 0.975 -4.287821) (width 0.25) (layer F.Cu) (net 20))
 (segment (start 1.625 -3.6) (end 1.625 -4.30141) (width 0.25) (layer F.Cu) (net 19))
 (segment (start 1.625 -4.30141) (end 2.275 -4.95141) (width 0.25) (layer F.Cu) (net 19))
 (segment (start 2.275 -4.95141) (end 2.275 -8.6) (width 0.25) (layer F.Cu) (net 19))
 (segment (start -5.575 -2.25) (end -5.575 1.415) (width 0.25) (layer F.Cu) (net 8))
 (segment (start -6.225 2.065) (end -6.225 2.75) (width 0.25) (layer F.Cu) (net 8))
 (segment (start -5.575 1.415) (end -6.225 2.065) (width 0.25) (layer F.Cu) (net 8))
 (segment (start -6.875 2.073157) (end -6.875 2.75) (width 0.25) (layer F.Cu) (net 4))
 (segment (start -6.225 1.423157) (end -6.875 2.073157) (width 0.25) (layer F.Cu) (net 4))
 (segment (start -6.225 -2.25) (end -6.225 1.423157) (width 0.25) (layer F.Cu) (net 4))
 (segment (start -6.875 1.423157) (end -7.525 2.073157) (width 0.25) (layer F.Cu) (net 5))
 (segment (start -7.525 2.073157) (end -7.525 2.75) (width 0.25) (layer F.Cu) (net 5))
 (segment (start -6.875 -2.25) (end -6.875 1.423157) (width 0.25) (layer F.Cu) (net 5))
 (segment (start -8.175 2.073157) (end -8.175 2.75) (width 0.25) (layer F.Cu) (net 6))
 (segment (start -7.525 1.423157) (end -8.175 2.073157) (width 0.25) (layer F.Cu) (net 6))
 (segment (start -7.525 -2.25) (end -7.525 1.423157) (width 0.25) (layer F.Cu) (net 6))
 (segment (start 2.925 -8.6) (end 2.925 -4.965) (width 0.25) (layer F.Cu) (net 18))
 (segment (start 2.275 -4.315) (end 2.275 -3.6) (width 0.25) (layer F.Cu) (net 18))
 (segment (start 2.925 -4.965) (end 2.275 -4.315) (width 0.25) (layer F.Cu) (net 18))
 (segment (start -8.825 2.073157) (end -8.825 2.75) (width 0.25) (layer F.Cu) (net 1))
 (segment (start -8.175 1.423157) (end -8.825 2.073157) (width 0.25) (layer F.Cu) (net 1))
 (segment (start -8.175 -2.25) (end -8.175 1.423157) (width 0.25) (layer F.Cu) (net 1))
 (segment (start -9.475 2.073157) (end -9.475 2.75) (width 0.25) (layer F.Cu) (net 3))
 (segment (start -8.825 1.423157) (end -9.475 2.073157) (width 0.25) (layer F.Cu) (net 3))
 (segment (start -8.825 -2.25) (end -8.825 1.423157) (width 0.25) (layer F.Cu) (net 3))
 (segment (start -10.125 2.073157) (end -10.125 2.75) (width 0.25) (layer F.Cu) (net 7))
 (segment (start -9.475 1.423157) (end -10.125 2.073157) (width 0.25) (layer F.Cu) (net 7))
 (segment (start -9.475 -2.25) (end -9.475 1.423157) (width 0.25) (layer F.Cu) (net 7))
 (segment (start -10.125 -2.25) (end -10.125 1.436747) (width 0.25) (layer F.Cu) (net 2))
 (segment (start -10.775 2.073157) (end -10.775 2.75) (width 0.25) (layer F.Cu) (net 2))
 (segment (start -10.13859 1.436747) (end -10.775 2.073157) (width 0.25) (layer F.Cu) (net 2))
 (segment (start -10.125 1.436747) (end -10.13859 1.436747) (width 0.25) (layer F.Cu) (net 2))
 (segment (start -5.575 -8.6) (end -5.575 -4.935) (width 0.25) (layer F.Cu) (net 13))
 (segment (start -6.225 -4.285) (end -6.225 -3.6) (width 0.25) (layer F.Cu) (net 13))
 (segment (start -5.575 -4.935) (end -6.225 -4.285) (width 0.25) (layer F.Cu) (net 13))
 (segment (start -6.875 -4.276843) (end -6.875 -3.6) (width 0.25) (layer F.Cu) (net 16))
 (segment (start -6.225 -4.926843) (end -6.875 -4.276843) (width 0.25) (layer F.Cu) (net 16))
 (segment (start -6.225 -8.6) (end -6.225 -4.926843) (width 0.25) (layer F.Cu) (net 16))
 (segment (start -7.525 -4.276843) (end -7.525 -3.6) (width 0.25) (layer F.Cu) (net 14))
 (segment (start -6.875 -4.926843) (end -7.525 -4.276843) (width 0.25) (layer F.Cu) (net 14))
 (segment (start -6.875 -8.6) (end -6.875 -4.926843) (width 0.25) (layer F.Cu) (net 14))
 (segment (start -8.175 -4.276843) (end -8.175 -3.6) (width 0.25) (layer F.Cu) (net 15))
 (segment (start -7.525 -4.926843) (end -8.175 -4.276843) (width 0.25) (layer F.Cu) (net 15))
 (segment (start -7.525 -8.6) (end -7.525 -4.926843) (width 0.25) (layer F.Cu) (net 15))
 (segment (start -8.825 -4.276843) (end -8.825 -3.6) (width 0.25) (layer F.Cu) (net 12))
 (segment (start -8.175 -4.926843) (end -8.825 -4.276843) (width 0.25) (layer F.Cu) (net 12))
 (segment (start -8.175 -8.6) (end -8.175 -4.926843) (width 0.25) (layer F.Cu) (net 12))
 (segment (start -9.475 -4.276843) (end -9.475 -3.6) (width 0.25) (layer F.Cu) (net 9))
 (segment (start -8.825 -4.926843) (end -9.475 -4.276843) (width 0.25) (layer F.Cu) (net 9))
 (segment (start -8.825 -8.6) (end -8.825 -4.926843) (width 0.25) (layer F.Cu) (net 9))
 (segment (start -10.125 -4.276843) (end -10.125 -3.6) (width 0.25) (layer F.Cu) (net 10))
 (segment (start -9.475 -4.926843) (end -10.125 -4.276843) (width 0.25) (layer F.Cu) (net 10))
 (segment (start -9.475 -8.6) (end -9.475 -4.926843) (width 0.25) (layer F.Cu) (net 10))
 (segment (start -10.125 -8.6) (end -10.125 -5.075) (width 0.25) (layer F.Cu) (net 11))
 (segment (start -10.775 -4.425) (end -10.775 -3.6) (width 0.25) (layer F.Cu) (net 11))
 (segment (start -10.125 -5.075) (end -10.775 -4.425) (width 0.25) (layer F.Cu) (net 11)))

